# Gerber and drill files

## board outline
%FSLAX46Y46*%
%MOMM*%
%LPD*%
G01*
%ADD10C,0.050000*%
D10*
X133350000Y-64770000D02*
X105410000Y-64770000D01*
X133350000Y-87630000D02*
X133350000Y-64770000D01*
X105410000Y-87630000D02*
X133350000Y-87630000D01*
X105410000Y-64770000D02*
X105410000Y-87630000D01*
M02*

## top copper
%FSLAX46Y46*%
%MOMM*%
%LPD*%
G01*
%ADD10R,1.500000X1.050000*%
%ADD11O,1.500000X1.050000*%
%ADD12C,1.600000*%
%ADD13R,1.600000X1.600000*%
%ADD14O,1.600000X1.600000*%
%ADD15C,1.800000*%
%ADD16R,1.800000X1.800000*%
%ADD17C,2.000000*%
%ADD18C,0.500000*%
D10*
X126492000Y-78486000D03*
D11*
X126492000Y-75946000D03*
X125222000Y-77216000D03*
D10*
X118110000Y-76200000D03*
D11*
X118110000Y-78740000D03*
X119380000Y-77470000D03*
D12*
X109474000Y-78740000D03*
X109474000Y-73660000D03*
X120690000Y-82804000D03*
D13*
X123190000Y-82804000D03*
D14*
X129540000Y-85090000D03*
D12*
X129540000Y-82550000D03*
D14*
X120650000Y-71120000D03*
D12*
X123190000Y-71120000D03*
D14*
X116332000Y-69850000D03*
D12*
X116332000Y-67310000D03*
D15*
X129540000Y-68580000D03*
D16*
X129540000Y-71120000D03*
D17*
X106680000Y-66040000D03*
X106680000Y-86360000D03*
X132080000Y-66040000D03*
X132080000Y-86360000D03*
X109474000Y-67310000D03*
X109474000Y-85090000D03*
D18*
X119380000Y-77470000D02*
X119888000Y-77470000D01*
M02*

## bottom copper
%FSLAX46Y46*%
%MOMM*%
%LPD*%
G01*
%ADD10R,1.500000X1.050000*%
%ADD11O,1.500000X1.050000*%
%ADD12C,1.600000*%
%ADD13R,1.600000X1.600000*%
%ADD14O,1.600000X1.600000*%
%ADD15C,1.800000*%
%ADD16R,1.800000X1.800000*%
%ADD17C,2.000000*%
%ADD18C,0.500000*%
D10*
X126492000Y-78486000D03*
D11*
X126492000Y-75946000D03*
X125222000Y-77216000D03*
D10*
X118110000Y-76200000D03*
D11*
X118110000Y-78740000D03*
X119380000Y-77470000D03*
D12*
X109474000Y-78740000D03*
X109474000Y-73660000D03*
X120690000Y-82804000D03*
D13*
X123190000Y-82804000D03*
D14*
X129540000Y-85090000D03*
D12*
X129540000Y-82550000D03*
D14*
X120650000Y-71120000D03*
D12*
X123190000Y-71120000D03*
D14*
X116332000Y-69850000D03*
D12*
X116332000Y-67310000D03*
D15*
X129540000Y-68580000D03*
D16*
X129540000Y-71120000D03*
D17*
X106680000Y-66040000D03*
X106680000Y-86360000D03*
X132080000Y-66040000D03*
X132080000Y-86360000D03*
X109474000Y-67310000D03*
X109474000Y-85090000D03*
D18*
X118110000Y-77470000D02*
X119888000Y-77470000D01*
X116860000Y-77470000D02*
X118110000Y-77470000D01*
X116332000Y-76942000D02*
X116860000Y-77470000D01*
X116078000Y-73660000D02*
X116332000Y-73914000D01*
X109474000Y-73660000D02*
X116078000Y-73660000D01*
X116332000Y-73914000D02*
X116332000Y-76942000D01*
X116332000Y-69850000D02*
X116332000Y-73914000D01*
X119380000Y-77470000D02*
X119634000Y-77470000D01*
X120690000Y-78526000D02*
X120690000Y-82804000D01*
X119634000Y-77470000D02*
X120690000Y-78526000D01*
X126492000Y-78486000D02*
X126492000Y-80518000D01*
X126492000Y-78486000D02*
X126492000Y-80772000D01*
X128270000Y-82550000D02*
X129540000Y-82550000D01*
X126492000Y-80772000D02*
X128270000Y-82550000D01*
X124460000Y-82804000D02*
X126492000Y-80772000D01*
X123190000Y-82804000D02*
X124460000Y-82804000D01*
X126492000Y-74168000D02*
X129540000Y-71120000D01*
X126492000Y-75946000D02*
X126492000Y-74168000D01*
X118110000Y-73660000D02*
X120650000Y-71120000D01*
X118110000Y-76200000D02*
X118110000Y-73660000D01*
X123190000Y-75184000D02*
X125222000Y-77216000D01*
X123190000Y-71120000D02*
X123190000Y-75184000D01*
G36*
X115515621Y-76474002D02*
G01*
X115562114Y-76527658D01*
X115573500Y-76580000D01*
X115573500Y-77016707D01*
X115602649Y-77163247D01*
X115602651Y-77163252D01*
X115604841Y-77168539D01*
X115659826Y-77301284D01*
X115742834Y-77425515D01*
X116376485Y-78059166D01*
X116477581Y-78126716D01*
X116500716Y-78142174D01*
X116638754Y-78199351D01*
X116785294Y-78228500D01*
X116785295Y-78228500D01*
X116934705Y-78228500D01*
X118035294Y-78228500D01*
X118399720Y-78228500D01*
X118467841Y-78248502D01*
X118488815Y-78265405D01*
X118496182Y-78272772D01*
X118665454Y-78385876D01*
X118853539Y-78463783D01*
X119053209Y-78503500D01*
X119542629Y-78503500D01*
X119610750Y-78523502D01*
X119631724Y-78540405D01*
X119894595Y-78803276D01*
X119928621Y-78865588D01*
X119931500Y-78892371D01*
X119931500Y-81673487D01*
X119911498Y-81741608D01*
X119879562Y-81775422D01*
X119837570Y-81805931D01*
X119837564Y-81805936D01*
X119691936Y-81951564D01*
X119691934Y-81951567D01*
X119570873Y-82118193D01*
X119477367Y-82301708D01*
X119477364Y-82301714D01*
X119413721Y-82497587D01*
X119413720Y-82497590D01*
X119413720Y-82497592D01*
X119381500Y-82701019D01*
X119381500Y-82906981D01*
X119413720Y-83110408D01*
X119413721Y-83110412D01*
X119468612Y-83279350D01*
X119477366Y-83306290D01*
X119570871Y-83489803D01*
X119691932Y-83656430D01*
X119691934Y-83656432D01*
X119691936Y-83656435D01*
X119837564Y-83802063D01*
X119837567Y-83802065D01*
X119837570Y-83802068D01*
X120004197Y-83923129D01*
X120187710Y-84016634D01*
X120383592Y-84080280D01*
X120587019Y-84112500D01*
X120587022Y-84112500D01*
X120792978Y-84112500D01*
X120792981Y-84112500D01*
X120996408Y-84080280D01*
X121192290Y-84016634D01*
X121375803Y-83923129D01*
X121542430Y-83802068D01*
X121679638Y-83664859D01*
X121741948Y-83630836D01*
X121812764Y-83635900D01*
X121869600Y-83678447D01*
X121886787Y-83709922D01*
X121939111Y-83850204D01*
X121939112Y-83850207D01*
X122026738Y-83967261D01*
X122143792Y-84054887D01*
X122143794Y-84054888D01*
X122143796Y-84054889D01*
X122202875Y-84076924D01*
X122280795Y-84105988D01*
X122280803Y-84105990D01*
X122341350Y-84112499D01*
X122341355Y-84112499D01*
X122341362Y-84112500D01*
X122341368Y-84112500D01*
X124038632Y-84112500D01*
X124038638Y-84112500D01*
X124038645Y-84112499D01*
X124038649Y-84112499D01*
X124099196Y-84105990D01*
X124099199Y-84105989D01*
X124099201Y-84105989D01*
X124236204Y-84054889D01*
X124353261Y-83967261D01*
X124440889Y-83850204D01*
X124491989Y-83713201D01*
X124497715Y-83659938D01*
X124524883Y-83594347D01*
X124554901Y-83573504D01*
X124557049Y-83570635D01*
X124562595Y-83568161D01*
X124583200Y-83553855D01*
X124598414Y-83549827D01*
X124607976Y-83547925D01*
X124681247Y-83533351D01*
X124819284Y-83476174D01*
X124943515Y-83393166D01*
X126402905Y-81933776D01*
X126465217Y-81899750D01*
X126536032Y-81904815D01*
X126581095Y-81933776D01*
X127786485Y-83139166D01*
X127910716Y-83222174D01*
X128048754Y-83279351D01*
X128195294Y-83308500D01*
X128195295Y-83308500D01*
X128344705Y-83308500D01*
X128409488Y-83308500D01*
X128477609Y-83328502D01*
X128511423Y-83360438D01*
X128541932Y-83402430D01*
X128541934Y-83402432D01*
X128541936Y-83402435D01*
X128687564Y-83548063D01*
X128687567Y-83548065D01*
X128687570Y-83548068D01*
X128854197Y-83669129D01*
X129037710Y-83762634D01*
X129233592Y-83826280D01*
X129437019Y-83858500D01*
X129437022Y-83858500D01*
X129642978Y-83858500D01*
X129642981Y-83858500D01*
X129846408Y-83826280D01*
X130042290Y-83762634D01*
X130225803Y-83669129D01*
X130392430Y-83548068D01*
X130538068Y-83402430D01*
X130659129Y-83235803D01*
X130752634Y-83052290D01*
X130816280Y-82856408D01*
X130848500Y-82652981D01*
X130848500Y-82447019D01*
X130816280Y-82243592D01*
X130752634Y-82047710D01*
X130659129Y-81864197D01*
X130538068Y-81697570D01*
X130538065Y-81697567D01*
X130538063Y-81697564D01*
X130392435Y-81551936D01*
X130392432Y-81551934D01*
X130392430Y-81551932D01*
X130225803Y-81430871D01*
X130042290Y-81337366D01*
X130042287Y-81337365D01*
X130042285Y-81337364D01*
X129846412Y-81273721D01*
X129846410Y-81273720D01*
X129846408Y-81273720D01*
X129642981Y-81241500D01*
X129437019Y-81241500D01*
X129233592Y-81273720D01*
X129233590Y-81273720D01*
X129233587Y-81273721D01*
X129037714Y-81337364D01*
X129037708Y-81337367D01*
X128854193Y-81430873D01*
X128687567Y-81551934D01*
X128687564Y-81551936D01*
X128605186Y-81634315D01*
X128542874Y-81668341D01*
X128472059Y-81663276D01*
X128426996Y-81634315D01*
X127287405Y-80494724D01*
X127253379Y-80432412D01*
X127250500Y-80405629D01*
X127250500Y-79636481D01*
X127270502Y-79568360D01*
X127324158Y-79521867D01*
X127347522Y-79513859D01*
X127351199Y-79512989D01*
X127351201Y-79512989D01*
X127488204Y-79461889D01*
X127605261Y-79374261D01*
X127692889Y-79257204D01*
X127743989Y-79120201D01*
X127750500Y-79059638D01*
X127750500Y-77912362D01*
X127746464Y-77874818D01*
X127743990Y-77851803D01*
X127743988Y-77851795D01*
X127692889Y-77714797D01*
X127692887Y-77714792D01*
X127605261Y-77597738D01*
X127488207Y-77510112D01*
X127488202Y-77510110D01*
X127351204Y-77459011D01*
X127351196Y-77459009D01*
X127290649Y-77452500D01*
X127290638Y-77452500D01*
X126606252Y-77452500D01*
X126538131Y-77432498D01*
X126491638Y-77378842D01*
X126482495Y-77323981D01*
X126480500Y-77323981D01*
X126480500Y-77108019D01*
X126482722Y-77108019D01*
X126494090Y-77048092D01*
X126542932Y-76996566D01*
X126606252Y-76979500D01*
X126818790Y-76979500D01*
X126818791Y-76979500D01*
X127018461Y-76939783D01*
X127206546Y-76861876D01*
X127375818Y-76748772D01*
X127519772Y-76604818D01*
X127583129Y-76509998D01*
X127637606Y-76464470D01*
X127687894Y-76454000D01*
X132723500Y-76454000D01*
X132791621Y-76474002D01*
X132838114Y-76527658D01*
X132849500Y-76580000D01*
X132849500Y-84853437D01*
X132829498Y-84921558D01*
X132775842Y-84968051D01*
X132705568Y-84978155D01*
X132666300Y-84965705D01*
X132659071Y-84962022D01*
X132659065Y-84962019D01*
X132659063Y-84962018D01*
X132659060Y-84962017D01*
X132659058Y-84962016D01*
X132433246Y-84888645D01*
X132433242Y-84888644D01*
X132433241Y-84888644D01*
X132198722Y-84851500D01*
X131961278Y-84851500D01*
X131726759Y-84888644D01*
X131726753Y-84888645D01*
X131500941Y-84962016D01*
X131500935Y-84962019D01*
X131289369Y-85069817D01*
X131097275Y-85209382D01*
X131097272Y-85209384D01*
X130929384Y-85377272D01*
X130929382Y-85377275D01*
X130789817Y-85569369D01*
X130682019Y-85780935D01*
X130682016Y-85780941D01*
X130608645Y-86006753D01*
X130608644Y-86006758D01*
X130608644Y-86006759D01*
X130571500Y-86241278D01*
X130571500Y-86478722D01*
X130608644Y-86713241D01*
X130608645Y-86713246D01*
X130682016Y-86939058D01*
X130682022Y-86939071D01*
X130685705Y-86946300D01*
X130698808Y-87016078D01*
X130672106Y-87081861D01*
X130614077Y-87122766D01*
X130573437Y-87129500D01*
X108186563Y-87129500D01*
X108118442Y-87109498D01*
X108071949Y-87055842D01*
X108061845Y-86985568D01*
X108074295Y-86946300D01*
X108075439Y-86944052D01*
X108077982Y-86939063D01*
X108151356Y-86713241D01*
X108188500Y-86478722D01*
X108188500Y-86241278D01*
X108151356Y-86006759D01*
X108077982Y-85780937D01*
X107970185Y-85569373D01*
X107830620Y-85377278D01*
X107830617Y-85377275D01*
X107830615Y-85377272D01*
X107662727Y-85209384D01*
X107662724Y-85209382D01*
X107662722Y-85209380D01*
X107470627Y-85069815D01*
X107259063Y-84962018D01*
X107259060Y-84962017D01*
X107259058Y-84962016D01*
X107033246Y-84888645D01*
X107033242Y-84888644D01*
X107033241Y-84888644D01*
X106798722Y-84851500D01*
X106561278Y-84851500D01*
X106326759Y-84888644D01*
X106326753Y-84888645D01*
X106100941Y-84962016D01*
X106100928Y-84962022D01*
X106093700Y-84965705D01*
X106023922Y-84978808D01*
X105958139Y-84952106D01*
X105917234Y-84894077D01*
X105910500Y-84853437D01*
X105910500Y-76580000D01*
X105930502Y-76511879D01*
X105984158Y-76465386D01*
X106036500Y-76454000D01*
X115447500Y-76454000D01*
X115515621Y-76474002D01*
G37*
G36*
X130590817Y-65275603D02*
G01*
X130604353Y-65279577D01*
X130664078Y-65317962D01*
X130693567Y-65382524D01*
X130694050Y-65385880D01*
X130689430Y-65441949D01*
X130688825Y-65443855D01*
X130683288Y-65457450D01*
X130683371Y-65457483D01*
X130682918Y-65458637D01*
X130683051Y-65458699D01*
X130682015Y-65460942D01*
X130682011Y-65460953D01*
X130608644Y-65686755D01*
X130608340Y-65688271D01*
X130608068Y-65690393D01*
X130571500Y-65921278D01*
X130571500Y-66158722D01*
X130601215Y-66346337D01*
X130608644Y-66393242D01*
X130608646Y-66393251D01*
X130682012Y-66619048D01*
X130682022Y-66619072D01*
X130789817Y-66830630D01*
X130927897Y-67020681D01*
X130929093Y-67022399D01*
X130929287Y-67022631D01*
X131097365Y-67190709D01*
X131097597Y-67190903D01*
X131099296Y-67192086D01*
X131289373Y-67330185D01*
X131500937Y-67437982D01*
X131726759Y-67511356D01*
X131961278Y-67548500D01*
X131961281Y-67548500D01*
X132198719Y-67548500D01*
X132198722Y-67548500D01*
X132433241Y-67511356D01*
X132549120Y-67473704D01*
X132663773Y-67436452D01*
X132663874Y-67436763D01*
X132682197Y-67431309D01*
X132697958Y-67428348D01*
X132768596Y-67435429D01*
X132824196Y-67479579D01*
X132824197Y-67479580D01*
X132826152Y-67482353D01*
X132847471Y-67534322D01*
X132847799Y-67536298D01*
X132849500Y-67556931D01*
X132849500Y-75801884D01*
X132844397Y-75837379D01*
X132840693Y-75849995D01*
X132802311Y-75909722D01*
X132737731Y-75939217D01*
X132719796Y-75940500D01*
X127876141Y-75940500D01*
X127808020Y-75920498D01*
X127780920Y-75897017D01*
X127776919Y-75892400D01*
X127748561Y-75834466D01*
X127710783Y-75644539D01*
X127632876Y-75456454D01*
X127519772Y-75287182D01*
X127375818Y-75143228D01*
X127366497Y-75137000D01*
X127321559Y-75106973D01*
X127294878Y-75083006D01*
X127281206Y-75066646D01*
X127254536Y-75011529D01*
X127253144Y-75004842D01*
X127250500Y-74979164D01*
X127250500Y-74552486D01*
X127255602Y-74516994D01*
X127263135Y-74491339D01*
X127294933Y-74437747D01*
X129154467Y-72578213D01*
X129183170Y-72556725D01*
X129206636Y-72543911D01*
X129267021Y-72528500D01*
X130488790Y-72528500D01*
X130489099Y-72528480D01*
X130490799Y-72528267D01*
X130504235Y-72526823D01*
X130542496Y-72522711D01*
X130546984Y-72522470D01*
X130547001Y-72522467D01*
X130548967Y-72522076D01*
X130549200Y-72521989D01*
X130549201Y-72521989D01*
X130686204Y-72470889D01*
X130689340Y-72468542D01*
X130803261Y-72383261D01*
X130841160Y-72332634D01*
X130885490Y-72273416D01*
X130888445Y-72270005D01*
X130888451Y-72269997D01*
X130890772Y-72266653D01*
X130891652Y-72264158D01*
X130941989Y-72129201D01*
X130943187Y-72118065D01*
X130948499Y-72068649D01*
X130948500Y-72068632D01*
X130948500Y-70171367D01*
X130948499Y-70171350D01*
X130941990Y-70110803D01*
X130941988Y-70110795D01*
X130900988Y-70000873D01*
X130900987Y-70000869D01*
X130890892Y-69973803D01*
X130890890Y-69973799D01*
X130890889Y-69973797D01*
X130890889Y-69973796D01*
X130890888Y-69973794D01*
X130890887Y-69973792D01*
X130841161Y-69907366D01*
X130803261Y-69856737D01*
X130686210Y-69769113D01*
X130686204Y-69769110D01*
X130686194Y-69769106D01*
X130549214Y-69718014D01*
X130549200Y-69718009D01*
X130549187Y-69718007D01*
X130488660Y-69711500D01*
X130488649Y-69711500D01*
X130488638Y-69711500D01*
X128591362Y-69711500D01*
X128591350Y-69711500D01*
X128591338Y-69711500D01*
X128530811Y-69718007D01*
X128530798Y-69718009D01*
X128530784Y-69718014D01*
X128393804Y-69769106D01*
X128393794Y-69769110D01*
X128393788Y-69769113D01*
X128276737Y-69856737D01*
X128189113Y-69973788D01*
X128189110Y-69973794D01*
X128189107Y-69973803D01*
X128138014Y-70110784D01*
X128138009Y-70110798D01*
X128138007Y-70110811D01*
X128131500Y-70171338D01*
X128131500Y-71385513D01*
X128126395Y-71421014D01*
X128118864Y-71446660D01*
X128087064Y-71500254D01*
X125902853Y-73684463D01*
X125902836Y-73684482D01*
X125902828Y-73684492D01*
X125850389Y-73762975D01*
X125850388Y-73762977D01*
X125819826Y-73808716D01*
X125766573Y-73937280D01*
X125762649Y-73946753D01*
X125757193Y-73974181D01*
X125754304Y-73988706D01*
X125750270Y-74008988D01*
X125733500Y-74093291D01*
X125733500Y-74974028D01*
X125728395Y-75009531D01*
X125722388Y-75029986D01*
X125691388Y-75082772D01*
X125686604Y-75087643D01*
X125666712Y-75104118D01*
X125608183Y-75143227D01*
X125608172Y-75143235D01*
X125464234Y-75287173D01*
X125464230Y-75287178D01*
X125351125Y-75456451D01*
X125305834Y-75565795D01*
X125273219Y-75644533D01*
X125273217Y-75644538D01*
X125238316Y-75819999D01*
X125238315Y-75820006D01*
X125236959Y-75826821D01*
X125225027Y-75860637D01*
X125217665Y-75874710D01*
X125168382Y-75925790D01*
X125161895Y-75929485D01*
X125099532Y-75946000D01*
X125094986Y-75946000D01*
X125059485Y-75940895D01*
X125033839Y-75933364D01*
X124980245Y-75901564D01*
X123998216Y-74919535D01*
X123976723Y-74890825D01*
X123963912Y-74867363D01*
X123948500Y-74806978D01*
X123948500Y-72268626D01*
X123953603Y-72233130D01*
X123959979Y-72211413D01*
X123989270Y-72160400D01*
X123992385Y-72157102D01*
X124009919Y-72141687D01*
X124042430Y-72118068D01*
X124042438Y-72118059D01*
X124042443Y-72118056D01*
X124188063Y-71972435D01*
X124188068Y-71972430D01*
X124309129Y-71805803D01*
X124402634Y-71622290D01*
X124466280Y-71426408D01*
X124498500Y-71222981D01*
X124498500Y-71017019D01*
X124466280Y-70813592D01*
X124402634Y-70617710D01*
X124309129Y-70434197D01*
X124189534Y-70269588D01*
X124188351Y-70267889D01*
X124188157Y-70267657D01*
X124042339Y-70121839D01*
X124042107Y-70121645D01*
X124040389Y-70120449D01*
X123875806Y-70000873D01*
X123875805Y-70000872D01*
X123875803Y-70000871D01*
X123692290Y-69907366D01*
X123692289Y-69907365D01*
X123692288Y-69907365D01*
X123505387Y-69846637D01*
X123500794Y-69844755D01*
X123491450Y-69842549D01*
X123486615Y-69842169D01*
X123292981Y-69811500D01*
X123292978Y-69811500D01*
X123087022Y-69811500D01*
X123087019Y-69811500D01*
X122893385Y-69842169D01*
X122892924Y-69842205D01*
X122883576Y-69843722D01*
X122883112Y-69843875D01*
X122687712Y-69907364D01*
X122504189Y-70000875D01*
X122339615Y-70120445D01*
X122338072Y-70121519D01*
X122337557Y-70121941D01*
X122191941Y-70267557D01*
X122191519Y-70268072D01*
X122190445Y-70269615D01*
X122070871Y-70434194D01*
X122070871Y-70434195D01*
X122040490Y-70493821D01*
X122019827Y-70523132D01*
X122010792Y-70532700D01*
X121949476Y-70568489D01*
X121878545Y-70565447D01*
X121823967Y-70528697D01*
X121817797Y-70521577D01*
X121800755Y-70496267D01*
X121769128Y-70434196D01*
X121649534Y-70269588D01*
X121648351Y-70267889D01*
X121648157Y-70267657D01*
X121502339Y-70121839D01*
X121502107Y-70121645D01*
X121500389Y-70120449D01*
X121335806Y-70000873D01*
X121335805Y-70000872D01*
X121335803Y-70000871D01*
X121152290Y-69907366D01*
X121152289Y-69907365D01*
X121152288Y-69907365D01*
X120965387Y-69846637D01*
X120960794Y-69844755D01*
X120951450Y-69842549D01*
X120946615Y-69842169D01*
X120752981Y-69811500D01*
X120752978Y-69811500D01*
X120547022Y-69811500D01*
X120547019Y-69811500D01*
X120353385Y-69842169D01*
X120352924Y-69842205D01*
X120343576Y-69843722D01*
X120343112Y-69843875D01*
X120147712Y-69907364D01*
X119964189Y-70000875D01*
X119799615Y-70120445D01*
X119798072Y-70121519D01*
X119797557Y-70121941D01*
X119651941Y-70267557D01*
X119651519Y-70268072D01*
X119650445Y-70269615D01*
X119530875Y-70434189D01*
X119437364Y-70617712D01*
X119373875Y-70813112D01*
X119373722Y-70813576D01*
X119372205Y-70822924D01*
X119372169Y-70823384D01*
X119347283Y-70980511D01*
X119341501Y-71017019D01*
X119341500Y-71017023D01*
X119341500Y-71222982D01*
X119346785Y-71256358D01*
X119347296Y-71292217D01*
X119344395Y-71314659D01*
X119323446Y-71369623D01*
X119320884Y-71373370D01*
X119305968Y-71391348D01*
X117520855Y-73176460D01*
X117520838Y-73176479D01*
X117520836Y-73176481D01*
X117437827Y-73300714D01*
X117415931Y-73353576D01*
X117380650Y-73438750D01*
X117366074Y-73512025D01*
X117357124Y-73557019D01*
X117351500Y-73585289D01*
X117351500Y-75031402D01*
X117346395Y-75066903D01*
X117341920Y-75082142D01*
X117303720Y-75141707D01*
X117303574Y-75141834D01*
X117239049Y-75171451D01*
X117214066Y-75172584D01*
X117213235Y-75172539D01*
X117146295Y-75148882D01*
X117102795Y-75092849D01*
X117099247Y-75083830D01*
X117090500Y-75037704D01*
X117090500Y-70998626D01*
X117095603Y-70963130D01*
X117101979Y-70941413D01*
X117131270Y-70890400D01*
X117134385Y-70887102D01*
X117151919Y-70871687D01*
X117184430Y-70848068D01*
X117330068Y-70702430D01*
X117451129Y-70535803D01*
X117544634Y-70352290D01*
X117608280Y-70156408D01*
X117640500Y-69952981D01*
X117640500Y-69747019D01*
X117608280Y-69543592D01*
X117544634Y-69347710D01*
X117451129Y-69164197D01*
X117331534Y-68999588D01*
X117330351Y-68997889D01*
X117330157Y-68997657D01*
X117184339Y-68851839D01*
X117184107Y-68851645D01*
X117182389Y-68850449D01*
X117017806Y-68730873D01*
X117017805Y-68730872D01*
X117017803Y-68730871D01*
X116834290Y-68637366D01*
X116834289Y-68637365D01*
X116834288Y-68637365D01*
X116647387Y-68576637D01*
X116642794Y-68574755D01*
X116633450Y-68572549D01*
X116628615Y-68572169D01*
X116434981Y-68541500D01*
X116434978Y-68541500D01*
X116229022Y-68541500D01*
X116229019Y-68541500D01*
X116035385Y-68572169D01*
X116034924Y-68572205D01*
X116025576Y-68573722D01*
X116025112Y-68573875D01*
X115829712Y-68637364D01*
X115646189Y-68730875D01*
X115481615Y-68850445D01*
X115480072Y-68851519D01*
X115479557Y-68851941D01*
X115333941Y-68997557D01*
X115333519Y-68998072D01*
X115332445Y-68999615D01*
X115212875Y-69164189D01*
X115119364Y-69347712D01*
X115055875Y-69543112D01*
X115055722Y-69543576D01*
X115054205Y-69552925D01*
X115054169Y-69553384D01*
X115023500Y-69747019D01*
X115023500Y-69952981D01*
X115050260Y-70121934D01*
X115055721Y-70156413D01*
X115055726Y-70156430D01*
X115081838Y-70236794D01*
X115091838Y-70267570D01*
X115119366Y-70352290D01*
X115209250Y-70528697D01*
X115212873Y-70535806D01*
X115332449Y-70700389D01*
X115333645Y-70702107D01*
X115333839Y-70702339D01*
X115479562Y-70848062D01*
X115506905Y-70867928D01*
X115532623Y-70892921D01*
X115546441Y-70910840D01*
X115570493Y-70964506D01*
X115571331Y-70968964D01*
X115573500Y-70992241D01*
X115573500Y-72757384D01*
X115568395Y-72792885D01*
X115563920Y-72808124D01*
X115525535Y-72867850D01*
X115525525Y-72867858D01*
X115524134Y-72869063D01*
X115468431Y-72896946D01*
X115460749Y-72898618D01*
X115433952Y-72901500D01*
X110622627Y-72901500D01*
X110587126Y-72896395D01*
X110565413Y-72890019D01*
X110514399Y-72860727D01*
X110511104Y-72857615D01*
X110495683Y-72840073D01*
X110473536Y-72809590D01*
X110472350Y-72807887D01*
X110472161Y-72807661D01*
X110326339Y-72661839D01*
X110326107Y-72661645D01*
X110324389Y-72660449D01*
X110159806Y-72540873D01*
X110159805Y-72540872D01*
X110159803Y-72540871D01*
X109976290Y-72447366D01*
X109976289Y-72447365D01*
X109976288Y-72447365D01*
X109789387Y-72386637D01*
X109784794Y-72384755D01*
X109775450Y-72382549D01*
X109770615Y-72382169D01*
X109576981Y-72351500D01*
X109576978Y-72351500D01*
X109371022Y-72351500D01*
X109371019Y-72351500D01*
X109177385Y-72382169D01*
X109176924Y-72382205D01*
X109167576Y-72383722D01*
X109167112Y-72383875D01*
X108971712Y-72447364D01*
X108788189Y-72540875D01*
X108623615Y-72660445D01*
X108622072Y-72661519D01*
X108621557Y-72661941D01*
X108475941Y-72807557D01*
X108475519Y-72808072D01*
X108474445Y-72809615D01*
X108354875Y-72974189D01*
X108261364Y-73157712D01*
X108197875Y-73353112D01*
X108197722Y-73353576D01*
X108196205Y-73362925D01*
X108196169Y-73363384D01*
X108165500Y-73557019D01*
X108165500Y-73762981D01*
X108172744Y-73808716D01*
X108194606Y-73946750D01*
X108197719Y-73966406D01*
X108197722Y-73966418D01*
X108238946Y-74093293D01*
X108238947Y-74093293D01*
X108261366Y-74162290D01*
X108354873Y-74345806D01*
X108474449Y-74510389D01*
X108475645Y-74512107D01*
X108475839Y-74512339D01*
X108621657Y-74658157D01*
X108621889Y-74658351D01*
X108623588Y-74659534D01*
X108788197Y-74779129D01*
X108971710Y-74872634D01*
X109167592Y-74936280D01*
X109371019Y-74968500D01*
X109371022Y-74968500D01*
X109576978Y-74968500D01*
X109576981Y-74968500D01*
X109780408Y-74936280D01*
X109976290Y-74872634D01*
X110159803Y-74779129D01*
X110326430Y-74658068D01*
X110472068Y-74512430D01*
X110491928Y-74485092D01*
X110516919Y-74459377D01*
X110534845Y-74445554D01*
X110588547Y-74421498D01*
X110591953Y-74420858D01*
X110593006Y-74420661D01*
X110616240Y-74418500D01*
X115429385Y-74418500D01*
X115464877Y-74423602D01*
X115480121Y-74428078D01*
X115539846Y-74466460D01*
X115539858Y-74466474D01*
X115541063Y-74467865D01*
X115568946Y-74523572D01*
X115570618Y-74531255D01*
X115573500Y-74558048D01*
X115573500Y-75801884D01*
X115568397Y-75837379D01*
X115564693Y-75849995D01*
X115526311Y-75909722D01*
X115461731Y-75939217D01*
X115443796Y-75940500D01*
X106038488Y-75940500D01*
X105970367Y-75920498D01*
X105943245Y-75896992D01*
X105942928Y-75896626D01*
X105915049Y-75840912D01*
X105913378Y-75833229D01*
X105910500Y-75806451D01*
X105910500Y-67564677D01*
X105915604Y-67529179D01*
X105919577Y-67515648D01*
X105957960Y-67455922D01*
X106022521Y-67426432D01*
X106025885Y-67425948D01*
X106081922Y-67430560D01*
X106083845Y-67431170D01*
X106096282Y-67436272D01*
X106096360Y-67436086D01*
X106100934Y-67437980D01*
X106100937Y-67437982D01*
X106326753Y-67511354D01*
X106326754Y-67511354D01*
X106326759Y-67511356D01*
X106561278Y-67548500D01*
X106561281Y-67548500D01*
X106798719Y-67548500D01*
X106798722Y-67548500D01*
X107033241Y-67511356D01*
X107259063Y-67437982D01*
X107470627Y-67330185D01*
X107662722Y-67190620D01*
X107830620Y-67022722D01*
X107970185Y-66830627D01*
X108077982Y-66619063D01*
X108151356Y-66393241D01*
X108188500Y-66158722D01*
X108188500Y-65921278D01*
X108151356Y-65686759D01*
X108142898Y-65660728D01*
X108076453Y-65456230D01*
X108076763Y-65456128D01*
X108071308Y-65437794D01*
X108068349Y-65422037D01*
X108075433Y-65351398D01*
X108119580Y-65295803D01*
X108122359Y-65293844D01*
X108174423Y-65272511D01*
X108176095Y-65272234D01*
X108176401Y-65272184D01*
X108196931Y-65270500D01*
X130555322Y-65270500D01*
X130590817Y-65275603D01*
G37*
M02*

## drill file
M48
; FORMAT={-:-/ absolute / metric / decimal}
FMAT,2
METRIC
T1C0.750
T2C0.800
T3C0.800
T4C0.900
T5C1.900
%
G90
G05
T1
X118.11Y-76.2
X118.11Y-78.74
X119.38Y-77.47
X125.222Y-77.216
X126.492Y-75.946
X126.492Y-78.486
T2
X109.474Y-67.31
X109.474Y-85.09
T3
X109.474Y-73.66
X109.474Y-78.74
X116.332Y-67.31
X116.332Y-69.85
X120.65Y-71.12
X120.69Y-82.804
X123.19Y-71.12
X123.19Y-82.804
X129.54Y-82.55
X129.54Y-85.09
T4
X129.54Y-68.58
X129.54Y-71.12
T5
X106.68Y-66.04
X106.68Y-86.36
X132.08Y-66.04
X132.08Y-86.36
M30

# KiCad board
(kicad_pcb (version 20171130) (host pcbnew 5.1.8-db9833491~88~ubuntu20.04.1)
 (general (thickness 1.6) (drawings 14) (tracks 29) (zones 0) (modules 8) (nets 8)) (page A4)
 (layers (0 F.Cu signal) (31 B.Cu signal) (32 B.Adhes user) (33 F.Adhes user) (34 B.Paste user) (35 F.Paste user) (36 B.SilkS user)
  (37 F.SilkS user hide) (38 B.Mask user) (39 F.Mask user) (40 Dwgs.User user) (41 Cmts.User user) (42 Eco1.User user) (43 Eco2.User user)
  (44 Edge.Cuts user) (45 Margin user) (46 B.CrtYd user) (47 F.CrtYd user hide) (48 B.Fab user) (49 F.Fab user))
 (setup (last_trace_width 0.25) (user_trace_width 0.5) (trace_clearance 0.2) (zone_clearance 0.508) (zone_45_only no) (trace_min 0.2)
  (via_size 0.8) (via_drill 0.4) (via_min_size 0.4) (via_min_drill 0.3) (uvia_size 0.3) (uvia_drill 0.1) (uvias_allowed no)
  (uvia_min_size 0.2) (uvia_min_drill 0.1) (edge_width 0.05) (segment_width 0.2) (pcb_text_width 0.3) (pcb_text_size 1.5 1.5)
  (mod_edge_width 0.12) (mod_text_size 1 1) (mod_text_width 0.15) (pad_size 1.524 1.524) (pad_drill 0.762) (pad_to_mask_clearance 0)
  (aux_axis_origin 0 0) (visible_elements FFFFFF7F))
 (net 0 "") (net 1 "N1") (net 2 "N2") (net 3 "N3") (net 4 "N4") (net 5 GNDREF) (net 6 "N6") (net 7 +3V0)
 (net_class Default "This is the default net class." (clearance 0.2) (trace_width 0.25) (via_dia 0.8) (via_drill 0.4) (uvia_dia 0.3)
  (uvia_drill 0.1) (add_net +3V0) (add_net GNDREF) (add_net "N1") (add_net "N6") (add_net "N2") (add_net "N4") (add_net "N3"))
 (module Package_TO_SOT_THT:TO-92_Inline (layer F.Cu) (at 126.492 78.486 90)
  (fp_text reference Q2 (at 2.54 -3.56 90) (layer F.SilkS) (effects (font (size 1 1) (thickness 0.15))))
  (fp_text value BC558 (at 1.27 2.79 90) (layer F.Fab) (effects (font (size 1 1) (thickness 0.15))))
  (pad 1 thru_hole rect (at 0 0 90) (size 1.05 1.5) (drill 0.75) (layers *.Cu *.Mask) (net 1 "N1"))
  (pad 3 thru_hole oval (at 2.54 0 90) (size 1.05 1.5) (drill 0.75) (layers *.Cu *.Mask) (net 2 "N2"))
  (pad 2 thru_hole oval (at 1.27 -1.27 90) (size 1.05 1.5) (drill 0.75) (layers *.Cu *.Mask) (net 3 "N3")))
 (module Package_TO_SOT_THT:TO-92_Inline (layer F.Cu) (at 118.11 76.2 270)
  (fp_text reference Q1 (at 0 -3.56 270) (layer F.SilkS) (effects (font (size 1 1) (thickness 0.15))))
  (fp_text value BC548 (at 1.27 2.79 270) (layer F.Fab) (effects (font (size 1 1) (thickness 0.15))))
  (pad 1 thru_hole rect (at 0 0 270) (size 1.05 1.5) (drill 0.75) (layers *.Cu *.Mask) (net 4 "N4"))
  (pad 3 thru_hole oval (at 2.54 0 270) (size 1.05 1.5) (drill 0.75) (layers *.Cu *.Mask) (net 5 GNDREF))
  (pad 2 thru_hole oval (at 1.27 -1.27 270) (size 1.05 1.5) (drill 0.75) (layers *.Cu *.Mask) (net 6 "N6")))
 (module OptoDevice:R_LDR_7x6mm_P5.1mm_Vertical (layer F.Cu) (at 109.474 73.66 270)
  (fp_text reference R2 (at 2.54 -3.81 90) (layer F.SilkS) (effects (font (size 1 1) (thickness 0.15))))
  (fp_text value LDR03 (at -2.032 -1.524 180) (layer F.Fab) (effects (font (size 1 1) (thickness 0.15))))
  (pad 2 thru_hole circle (at 5.08 0 270) (size 1.6 1.6) (drill 0.8) (layers *.Cu *.Mask) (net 5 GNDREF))
  (pad 1 thru_hole circle (at 0 0 270) (size 1.6 1.6) (drill 0.8) (layers *.Cu *.Mask) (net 6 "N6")))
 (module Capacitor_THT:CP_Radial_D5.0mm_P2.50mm (layer F.Cu) (at 123.19 82.804 180)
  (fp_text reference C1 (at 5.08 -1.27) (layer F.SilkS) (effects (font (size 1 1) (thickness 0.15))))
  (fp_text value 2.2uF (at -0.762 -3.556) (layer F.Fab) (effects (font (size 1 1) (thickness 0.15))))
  (pad 2 thru_hole circle (at 2.5 0 180) (size 1.6 1.6) (drill 0.8) (layers *.Cu *.Mask) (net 6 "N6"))
  (pad 1 thru_hole rect (at 0 0 180) (size 1.6 1.6) (drill 0.8) (layers *.Cu *.Mask) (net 1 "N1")))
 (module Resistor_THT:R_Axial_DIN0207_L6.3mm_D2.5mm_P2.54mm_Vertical (layer F.Cu) (at 129.54 82.55 270)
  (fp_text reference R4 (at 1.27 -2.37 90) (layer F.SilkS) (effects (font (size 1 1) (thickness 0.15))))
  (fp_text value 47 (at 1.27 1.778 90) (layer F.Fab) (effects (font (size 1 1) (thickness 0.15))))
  (pad 2 thru_hole oval (at 2.54 0 270) (size 1.6 1.6) (drill 0.8) (layers *.Cu *.Mask) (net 5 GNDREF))
  (pad 1 thru_hole circle (at 0 0 270) (size 1.6 1.6) (drill 0.8) (layers *.Cu *.Mask) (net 1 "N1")))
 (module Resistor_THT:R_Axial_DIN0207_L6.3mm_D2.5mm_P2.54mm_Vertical (layer F.Cu) (at 123.19 71.12 180)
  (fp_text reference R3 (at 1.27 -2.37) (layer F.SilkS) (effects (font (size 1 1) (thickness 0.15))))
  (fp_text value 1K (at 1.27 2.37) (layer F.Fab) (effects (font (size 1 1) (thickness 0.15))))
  (pad 2 thru_hole oval (at 2.54 0 180) (size 1.6 1.6) (drill 0.8) (layers *.Cu *.Mask) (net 4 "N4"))
  (pad 1 thru_hole circle (at 0 0 180) (size 1.6 1.6) (drill 0.8) (layers *.Cu *.Mask) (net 3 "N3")))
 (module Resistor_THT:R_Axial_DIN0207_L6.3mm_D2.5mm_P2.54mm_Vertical (layer F.Cu) (at 116.332 67.31 270)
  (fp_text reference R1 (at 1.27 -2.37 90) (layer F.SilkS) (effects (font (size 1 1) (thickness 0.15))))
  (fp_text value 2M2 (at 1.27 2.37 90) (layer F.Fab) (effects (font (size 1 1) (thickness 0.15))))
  (pad 2 thru_hole oval (at 2.54 0 270) (size 1.6 1.6) (drill 0.8) (layers *.Cu *.Mask) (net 6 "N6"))
  (pad 1 thru_hole circle (at 0 0 270) (size 1.6 1.6) (drill 0.8) (layers *.Cu *.Mask) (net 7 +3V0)))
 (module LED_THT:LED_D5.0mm (layer F.Cu) (at 129.54 71.12 90)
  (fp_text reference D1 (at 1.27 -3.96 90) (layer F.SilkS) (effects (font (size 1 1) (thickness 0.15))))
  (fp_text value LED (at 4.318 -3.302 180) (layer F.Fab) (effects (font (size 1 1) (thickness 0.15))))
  (pad 2 thru_hole circle (at 2.54 0 90) (size 1.8 1.8) (drill 0.9) (layers *.Cu *.Mask) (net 7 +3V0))
  (pad 1 thru_hole rect (at 0 0 90) (size 1.8 1.8) (drill 0.9) (layers *.Cu *.Mask) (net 2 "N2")))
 (gr_line (start 133.35 64.77) (end 105.41 64.77) (layer Edge.Cuts) (width 0.05))
 (gr_line (start 133.35 87.63) (end 133.35 64.77) (layer Edge.Cuts) (width 0.05))
 (gr_line (start 105.41 87.63) (end 133.35 87.63) (layer Edge.Cuts) (width 0.05))
 (gr_line (start 105.41 64.77) (end 105.41 87.63) (layer Edge.Cuts) (width 0.05))
 (via (at 106.68 66.04) (size 2) (drill 1.9) (layers F.Cu B.Cu) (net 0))
 (via (at 106.68 86.36) (size 2) (drill 1.9) (layers F.Cu B.Cu) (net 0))
 (via (at 132.08 66.04) (size 2) (drill 1.9) (layers F.Cu B.Cu) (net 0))
 (via (at 132.08 86.36) (size 2) (drill 1.9) (layers F.Cu B.Cu) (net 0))
 (segment (start 118.11 77.47) (end 119.888 77.47) (width 0.5) (layer B.Cu) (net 6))
 (segment (start 116.86 77.47) (end 118.11 77.47) (width 0.5) (layer B.Cu) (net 6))
 (segment (start 116.332 76.942) (end 116.86 77.47) (width 0.5) (layer B.Cu) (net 6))
 (segment (start 116.078 73.66) (end 116.332 73.914) (width 0.5) (layer B.Cu) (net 6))
 (segment (start 109.474 73.66) (end 116.078 73.66) (width 0.5) (layer B.Cu) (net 6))
 (segment (start 116.332 73.914) (end 116.332 76.942) (width 0.5) (layer B.Cu) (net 6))
 (segment (start 116.332 69.85) (end 116.332 73.914) (width 0.5) (layer B.Cu) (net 6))
 (segment (start 119.38 77.47) (end 119.888 77.47) (width 0.5) (layer F.Cu) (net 6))
 (segment (start 119.38 77.47) (end 119.634 77.47) (width 0.5) (layer B.Cu) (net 6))
 (segment (start 120.69 78.526) (end 120.69 82.804) (width 0.5) (layer B.Cu) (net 6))
 (segment (start 119.634 77.47) (end 120.69 78.526) (width 0.5) (layer B.Cu) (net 6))
 (segment (start 126.492 78.486) (end 126.492 80.518) (width 0.5) (layer B.Cu) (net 1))
 (segment (start 126.492 78.486) (end 126.492 80.772) (width 0.5) (layer B.Cu) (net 1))
 (segment (start 128.27 82.55) (end 129.54 82.55) (width 0.5) (layer B.Cu) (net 1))
 (segment (start 126.492 80.772) (end 128.27 82.55) (width 0.5) (layer B.Cu) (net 1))
 (segment (start 124.46 82.804) (end 126.492 80.772) (width 0.5) (layer B.Cu) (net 1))
 (segment (start 123.19 82.804) (end 124.46 82.804) (width 0.5) (layer B.Cu) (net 1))
 (segment (start 126.492 74.168) (end 129.54 71.12) (width 0.5) (layer B.Cu) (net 2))
 (segment (start 126.492 75.946) (end 126.492 74.168) (width 0.5) (layer B.Cu) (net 2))
 (segment (start 118.11 73.66) (end 120.65 71.12) (width 0.5) (layer B.Cu) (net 4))
 (segment (start 118.11 76.2) (end 118.11 73.66) (width 0.5) (layer B.Cu) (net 4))
 (segment (start 123.19 75.184) (end 125.222 77.216) (width 0.5) (layer B.Cu) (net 3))
 (segment (start 123.19 71.12) (end 123.19 75.184) (width 0.5) (layer B.Cu) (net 3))
 (via (at 109.474 67.31) (size 2) (drill 0.8) (layers F.Cu B.Cu) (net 7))
 (via (at 109.474 85.09) (size 2) (drill 0.8) (layers F.Cu B.Cu) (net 5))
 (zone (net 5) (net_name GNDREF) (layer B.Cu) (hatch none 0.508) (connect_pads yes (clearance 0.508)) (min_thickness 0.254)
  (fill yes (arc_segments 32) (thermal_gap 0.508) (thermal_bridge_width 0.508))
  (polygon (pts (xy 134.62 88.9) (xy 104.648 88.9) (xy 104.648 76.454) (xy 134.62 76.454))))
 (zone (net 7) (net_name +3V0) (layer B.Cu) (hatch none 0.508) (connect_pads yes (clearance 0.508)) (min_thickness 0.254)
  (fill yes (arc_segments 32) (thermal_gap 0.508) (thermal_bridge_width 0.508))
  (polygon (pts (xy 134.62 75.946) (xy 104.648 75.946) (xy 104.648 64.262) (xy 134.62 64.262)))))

